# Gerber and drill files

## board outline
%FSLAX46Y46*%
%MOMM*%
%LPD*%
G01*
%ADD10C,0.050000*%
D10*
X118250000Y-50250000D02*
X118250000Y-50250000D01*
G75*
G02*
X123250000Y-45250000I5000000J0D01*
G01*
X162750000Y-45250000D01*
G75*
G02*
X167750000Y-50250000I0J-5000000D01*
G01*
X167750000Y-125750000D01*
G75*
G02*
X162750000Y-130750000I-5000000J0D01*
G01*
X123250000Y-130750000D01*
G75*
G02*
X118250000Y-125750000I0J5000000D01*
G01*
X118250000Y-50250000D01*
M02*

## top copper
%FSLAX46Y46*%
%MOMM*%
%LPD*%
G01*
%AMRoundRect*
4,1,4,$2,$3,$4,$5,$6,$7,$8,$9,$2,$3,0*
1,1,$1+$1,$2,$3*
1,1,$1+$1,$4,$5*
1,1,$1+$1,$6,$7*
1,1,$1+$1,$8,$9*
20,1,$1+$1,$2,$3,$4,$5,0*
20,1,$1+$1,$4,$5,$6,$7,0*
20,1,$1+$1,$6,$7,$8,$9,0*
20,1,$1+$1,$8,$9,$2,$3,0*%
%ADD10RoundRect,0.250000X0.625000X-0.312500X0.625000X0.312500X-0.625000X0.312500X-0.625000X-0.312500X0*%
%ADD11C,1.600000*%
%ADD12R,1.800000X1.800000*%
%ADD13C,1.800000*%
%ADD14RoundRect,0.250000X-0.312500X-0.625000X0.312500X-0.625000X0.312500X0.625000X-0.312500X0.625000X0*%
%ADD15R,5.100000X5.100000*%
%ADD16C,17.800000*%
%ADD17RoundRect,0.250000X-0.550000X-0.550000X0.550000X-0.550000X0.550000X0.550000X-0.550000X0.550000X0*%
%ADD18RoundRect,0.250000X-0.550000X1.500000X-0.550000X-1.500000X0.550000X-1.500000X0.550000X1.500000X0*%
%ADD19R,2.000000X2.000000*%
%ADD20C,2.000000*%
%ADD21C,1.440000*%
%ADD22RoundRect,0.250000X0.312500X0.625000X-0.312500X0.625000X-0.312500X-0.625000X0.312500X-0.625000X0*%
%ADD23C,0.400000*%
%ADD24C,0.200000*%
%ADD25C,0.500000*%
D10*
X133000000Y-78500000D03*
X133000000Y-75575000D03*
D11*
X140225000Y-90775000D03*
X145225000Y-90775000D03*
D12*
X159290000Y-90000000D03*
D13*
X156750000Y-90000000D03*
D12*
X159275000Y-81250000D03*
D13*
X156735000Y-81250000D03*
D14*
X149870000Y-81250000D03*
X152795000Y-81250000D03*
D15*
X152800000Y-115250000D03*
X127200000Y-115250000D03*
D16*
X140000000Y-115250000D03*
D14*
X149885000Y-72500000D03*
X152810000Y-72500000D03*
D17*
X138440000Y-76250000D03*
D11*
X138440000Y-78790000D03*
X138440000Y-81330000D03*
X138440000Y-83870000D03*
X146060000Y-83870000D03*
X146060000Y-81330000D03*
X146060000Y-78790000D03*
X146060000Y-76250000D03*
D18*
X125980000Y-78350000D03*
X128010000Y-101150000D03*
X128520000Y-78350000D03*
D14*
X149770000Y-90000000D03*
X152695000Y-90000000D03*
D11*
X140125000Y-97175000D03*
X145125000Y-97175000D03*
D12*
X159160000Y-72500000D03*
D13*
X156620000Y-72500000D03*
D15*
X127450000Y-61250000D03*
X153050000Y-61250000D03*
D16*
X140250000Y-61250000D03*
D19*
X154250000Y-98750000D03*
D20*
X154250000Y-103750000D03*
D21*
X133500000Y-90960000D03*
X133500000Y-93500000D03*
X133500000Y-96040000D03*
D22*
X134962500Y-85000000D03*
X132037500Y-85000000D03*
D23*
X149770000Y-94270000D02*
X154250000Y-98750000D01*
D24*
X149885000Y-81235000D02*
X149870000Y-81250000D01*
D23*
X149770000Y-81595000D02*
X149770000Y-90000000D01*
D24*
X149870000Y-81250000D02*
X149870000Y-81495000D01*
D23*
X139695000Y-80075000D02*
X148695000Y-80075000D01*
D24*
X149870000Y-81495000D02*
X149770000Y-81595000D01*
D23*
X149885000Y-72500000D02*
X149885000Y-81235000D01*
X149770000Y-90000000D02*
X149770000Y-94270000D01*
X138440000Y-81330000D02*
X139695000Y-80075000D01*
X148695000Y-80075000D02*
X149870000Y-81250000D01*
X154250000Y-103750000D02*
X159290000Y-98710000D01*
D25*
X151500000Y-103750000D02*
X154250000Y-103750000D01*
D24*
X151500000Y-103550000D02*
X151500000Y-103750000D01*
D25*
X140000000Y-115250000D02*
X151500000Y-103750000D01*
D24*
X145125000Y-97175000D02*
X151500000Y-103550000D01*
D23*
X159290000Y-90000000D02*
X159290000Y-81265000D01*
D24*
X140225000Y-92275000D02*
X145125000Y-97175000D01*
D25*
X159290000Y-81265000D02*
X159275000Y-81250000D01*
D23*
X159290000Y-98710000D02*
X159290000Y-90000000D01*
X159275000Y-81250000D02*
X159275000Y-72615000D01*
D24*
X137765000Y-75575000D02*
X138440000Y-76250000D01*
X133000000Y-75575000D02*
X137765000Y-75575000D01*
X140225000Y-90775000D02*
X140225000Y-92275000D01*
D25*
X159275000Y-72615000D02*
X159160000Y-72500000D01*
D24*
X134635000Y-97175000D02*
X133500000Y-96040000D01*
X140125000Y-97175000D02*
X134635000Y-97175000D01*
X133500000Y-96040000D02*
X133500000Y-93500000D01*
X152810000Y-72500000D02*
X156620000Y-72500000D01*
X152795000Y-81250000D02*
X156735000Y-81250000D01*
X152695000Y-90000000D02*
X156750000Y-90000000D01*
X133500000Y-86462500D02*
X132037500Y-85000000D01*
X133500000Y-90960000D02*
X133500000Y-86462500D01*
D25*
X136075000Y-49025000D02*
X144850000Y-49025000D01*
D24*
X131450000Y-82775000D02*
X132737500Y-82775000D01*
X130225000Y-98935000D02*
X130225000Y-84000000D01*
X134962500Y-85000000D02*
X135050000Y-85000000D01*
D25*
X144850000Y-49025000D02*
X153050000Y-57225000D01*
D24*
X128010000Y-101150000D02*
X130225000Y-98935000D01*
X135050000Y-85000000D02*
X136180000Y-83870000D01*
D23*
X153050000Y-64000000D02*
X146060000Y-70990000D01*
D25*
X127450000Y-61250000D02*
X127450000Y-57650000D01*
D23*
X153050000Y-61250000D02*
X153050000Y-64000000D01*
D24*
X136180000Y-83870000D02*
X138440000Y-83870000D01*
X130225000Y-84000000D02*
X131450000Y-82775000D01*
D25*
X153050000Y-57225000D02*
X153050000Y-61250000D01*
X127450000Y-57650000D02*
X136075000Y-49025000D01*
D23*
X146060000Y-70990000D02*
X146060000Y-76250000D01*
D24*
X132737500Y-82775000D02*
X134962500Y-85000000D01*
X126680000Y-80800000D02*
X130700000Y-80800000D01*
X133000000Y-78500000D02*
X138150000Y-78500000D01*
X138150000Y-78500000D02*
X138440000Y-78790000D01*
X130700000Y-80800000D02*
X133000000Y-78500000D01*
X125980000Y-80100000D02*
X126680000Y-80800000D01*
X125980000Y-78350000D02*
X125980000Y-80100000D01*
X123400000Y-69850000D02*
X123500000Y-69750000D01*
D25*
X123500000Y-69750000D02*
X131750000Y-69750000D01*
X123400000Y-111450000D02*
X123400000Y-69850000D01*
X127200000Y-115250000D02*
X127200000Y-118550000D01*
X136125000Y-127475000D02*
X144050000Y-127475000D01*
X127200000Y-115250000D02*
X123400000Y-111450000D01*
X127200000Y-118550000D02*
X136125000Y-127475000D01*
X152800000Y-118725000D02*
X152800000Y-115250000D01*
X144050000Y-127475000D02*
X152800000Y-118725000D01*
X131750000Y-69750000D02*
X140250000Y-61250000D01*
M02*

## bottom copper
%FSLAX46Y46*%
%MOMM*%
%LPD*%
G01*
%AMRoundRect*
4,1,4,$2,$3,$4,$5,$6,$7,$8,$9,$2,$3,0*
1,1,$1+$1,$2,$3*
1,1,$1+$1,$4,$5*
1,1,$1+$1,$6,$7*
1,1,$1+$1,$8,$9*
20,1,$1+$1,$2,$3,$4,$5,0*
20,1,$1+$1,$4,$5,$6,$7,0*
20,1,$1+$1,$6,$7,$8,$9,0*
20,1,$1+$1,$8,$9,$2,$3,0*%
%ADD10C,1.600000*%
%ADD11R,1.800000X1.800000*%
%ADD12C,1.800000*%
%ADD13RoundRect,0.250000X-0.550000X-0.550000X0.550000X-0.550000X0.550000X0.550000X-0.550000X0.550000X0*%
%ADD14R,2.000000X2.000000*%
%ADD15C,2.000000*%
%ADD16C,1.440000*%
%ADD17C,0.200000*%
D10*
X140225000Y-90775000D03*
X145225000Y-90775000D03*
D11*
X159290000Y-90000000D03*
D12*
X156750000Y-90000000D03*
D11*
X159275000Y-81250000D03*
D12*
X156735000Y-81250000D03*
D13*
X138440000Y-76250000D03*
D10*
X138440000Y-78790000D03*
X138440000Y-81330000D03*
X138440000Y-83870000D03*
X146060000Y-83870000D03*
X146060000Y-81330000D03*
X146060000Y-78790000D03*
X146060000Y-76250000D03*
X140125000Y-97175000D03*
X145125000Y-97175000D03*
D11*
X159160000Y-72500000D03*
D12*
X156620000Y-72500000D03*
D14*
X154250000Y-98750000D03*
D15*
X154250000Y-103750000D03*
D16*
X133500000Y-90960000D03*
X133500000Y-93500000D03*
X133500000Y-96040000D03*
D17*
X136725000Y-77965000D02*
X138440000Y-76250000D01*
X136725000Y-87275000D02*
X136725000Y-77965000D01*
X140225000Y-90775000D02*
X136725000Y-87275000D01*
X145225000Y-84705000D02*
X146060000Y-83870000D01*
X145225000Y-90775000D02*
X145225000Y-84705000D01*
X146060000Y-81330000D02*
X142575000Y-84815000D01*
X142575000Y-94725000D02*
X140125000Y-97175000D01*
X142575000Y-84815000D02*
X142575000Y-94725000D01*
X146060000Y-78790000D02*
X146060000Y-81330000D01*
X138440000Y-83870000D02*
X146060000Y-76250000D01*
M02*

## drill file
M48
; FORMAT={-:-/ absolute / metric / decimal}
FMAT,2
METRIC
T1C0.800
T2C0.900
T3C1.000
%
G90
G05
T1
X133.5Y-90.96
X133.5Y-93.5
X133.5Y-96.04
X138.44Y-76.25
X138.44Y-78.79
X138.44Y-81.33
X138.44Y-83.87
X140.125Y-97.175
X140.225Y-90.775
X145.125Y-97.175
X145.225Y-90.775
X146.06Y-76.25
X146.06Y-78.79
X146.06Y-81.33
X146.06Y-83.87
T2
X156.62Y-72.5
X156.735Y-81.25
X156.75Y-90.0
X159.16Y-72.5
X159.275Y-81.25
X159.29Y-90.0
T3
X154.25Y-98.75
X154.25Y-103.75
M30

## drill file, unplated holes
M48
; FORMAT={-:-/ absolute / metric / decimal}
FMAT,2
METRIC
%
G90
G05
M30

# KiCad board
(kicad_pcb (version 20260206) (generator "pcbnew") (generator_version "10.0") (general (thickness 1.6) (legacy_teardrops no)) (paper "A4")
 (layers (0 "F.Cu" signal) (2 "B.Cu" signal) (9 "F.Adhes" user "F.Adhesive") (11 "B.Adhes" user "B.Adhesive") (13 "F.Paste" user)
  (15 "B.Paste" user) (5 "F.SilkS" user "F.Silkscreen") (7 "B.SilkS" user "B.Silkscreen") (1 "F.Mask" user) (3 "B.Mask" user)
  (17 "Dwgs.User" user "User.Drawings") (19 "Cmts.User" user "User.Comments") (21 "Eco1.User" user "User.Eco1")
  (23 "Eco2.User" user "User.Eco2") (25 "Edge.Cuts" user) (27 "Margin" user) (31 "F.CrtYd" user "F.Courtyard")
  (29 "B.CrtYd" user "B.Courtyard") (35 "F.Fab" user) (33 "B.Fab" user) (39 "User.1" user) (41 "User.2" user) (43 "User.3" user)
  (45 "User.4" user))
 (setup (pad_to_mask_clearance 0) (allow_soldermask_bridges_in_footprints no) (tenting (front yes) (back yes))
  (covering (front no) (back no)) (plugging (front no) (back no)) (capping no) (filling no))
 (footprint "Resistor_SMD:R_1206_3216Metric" (layer "F.Cu") (at 133 77.0375 90)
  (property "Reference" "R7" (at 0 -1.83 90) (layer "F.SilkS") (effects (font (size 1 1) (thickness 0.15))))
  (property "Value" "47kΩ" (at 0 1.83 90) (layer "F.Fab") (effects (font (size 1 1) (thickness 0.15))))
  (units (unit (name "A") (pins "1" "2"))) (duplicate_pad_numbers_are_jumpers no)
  (pad "1" smd roundrect (at -1.4625 0 90) (size 1.125 1.75) (layers "F.Cu" "F.Mask" "F.Paste") (roundrect_rratio 0.222222)
   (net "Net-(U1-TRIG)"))
  (pad "2" smd roundrect (at 1.4625 0 90) (size 1.125 1.75) (layers "F.Cu" "F.Mask" "F.Paste") (roundrect_rratio 0.222222) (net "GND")))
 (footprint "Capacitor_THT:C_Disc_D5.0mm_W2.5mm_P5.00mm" (layer "F.Cu") (at 140.225 90.775)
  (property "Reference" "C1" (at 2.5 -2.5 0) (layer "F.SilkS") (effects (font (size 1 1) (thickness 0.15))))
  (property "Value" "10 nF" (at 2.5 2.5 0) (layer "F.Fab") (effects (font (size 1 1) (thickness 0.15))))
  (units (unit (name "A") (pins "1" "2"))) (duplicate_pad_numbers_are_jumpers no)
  (pad "1" thru_hole circle (at 0 0) (size 1.6 1.6) (drill 0.8) (layers "*.Cu" "*.Mask") (remove_unused_layers no) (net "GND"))
  (pad "2" thru_hole circle (at 5 0) (size 1.6 1.6) (drill 0.8) (layers "*.Cu" "*.Mask") (remove_unused_layers no) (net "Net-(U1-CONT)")))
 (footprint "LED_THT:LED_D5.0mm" (layer "F.Cu") (at 159.29 90 180)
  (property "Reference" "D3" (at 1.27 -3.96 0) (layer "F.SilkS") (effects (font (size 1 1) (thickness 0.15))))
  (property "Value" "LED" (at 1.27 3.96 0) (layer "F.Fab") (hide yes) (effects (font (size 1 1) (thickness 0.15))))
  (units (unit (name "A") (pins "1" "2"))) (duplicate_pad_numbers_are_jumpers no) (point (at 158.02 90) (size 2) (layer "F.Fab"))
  (pad "1" thru_hole rect (at 0 0 180) (size 1.8 1.8) (drill 0.9) (layers "*.Cu" "*.Mask") (remove_unused_layers no) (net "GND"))
  (pad "2" thru_hole circle (at 2.54 0 180) (size 1.8 1.8) (drill 0.9) (layers "*.Cu" "*.Mask") (remove_unused_layers no) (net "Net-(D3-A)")))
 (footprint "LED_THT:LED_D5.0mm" (layer "F.Cu") (at 159.275 81.25 180)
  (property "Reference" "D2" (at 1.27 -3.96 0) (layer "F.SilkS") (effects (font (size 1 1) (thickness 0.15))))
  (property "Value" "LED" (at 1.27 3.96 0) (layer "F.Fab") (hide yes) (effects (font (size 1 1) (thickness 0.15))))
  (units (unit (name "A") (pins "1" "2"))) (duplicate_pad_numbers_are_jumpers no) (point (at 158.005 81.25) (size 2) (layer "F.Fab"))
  (pad "1" thru_hole rect (at 0 0 180) (size 1.8 1.8) (drill 0.9) (layers "*.Cu" "*.Mask") (remove_unused_layers no) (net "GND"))
  (pad "2" thru_hole circle (at 2.54 0 180) (size 1.8 1.8) (drill 0.9) (layers "*.Cu" "*.Mask") (remove_unused_layers no) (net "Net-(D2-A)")))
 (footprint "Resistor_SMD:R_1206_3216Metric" (layer "F.Cu") (at 151.3325 81.25)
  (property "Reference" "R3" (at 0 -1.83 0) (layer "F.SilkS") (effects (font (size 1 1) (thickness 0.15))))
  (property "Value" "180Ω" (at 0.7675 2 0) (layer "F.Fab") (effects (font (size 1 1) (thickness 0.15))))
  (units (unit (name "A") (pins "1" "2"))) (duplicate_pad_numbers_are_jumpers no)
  (pad "1" smd roundrect (at -1.4625 0) (size 1.125 1.75) (layers "F.Cu" "F.Mask" "F.Paste") (roundrect_rratio 0.222222) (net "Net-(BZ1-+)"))
  (pad "2" smd roundrect (at 1.4625 0) (size 1.125 1.75) (layers "F.Cu" "F.Mask" "F.Paste") (roundrect_rratio 0.222222) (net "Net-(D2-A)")))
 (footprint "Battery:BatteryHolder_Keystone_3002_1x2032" (layer "F.Cu") (at 140 115.25 180)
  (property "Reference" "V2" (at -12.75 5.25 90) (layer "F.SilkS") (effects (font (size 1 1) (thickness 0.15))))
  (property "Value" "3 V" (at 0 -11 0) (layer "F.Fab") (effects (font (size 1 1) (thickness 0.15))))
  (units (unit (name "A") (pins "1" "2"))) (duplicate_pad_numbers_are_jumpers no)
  (pad "1" smd rect (at -12.8 0 180) (size 5.1 5.1) (layers "F.Cu" "F.Mask" "F.Paste") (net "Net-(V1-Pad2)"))
  (pad "1" smd rect (at 12.8 0 180) (size 5.1 5.1) (layers "F.Cu" "F.Mask" "F.Paste") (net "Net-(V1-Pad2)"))
  (pad "2" smd circle (at 0 0 180) (size 17.8 17.8) (layers "F.Cu" "F.Mask") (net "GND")))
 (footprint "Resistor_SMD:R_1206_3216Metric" (layer "F.Cu") (at 151.3475 72.5)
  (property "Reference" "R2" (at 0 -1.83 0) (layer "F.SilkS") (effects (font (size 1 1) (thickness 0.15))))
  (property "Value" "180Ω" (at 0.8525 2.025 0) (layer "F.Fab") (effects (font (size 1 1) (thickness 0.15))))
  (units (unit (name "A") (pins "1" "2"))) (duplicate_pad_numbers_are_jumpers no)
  (pad "1" smd roundrect (at -1.4625 0) (size 1.125 1.75) (layers "F.Cu" "F.Mask" "F.Paste") (roundrect_rratio 0.222222) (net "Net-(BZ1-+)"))
  (pad "2" smd roundrect (at 1.4625 0) (size 1.125 1.75) (layers "F.Cu" "F.Mask" "F.Paste") (roundrect_rratio 0.222222) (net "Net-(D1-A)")))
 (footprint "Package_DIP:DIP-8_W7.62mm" (layer "F.Cu") (at 138.44 76.25)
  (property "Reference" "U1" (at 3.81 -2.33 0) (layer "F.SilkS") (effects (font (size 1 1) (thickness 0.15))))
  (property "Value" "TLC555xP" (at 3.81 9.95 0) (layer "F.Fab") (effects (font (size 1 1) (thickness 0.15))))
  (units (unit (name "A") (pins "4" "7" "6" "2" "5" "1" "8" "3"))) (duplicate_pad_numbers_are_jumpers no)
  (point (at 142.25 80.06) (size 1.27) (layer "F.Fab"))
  (pad "1" thru_hole roundrect (at 0 0) (size 1.6 1.6) (drill 0.8) (layers "*.Cu" "*.Mask") (remove_unused_layers no)
   (roundrect_rratio 0.15625) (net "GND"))
  (pad "2" thru_hole circle (at 0 2.54) (size 1.6 1.6) (drill 0.8) (layers "*.Cu" "*.Mask") (remove_unused_layers no) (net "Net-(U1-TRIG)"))
  (pad "3" thru_hole circle (at 0 5.08) (size 1.6 1.6) (drill 0.8) (layers "*.Cu" "*.Mask") (remove_unused_layers no) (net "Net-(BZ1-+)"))
  (pad "4" thru_hole circle (at 0 7.62) (size 1.6 1.6) (drill 0.8) (layers "*.Cu" "*.Mask") (remove_unused_layers no) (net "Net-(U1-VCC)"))
  (pad "5" thru_hole circle (at 7.62 7.62) (size 1.6 1.6) (drill 0.8) (layers "*.Cu" "*.Mask") (remove_unused_layers no)
   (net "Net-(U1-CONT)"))
  (pad "6" thru_hole circle (at 7.62 5.08) (size 1.6 1.6) (drill 0.8) (layers "*.Cu" "*.Mask") (remove_unused_layers no)
   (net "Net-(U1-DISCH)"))
  (pad "7" thru_hole circle (at 7.62 2.54) (size 1.6 1.6) (drill 0.8) (layers "*.Cu" "*.Mask") (remove_unused_layers no)
   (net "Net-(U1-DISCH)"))
  (pad "8" thru_hole circle (at 7.62 0) (size 1.6 1.6) (drill 0.8) (layers "*.Cu" "*.Mask") (remove_unused_layers no) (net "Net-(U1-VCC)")))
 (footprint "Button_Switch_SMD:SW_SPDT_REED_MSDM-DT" (layer "F.Cu") (at 128.01 89.75)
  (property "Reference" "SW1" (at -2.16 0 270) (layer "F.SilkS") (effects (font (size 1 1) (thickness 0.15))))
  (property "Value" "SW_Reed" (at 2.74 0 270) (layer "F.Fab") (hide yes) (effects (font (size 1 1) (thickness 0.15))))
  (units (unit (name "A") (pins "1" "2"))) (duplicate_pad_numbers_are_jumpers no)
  (pad "1" smd roundrect (at -2.03 -11.4 270) (size 3.5 1.6) (layers "F.Cu" "F.Mask" "F.Paste") (roundrect_rratio 0.15625)
   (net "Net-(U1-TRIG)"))
  (pad "2" smd roundrect (at 0 11.4 270) (size 3.5 1.6) (layers "F.Cu" "F.Mask" "F.Paste") (roundrect_rratio 0.15625) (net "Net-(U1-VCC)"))
  (pad "3" smd roundrect (at 0.51 -11.4 270) (size 3.5 1.6) (layers "F.Cu" "F.Mask" "F.Paste") (roundrect_rratio 0.15625)))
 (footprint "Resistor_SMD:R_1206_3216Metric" (layer "F.Cu") (at 151.2325 90)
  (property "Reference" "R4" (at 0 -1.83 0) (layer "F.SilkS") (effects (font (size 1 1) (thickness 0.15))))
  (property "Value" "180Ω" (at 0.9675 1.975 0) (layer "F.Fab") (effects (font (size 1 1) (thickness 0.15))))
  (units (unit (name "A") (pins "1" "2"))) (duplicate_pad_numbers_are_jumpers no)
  (pad "1" smd roundrect (at -1.4625 0) (size 1.125 1.75) (layers "F.Cu" "F.Mask" "F.Paste") (roundrect_rratio 0.222222) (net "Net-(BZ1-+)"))
  (pad "2" smd roundrect (at 1.4625 0) (size 1.125 1.75) (layers "F.Cu" "F.Mask" "F.Paste") (roundrect_rratio 0.222222) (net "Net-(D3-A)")))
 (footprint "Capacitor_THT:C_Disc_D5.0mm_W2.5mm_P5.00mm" (layer "F.Cu") (at 140.125 97.175)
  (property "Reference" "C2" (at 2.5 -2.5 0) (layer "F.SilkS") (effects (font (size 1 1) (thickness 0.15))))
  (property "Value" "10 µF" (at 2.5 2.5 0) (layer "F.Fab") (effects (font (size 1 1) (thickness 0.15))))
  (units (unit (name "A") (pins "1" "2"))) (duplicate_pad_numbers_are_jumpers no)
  (pad "1" thru_hole circle (at 0 0) (size 1.6 1.6) (drill 0.8) (layers "*.Cu" "*.Mask") (remove_unused_layers no) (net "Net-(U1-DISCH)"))
  (pad "2" thru_hole circle (at 5 0) (size 1.6 1.6) (drill 0.8) (layers "*.Cu" "*.Mask") (remove_unused_layers no) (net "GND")))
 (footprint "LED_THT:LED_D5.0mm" (layer "F.Cu") (at 159.16 72.5 180)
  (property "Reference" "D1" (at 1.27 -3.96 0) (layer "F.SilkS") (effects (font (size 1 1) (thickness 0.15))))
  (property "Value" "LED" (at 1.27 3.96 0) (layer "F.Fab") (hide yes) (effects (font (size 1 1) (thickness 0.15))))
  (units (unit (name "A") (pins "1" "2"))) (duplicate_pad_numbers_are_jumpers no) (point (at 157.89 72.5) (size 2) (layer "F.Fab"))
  (pad "1" thru_hole rect (at 0 0 180) (size 1.8 1.8) (drill 0.9) (layers "*.Cu" "*.Mask") (remove_unused_layers no) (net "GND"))
  (pad "2" thru_hole circle (at 2.54 0 180) (size 1.8 1.8) (drill 0.9) (layers "*.Cu" "*.Mask") (remove_unused_layers no) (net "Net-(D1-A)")))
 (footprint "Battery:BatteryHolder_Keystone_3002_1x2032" (layer "F.Cu") (at 140.25 61.25)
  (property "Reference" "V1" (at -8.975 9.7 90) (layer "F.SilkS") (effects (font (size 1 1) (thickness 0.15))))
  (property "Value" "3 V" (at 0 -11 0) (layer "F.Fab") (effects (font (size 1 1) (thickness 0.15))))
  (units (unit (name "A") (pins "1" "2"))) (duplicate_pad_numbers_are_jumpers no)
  (pad "1" smd rect (at -12.8 0) (size 5.1 5.1) (layers "F.Cu" "F.Mask" "F.Paste") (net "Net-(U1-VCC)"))
  (pad "1" smd rect (at 12.8 0) (size 5.1 5.1) (layers "F.Cu" "F.Mask" "F.Paste") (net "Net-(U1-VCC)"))
  (pad "2" smd circle (at 0 0) (size 17.8 17.8) (layers "F.Cu" "F.Mask") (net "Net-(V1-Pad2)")))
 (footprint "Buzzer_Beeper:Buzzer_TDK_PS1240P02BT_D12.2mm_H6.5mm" (layer "F.Cu") (at 154.25 98.75 -90)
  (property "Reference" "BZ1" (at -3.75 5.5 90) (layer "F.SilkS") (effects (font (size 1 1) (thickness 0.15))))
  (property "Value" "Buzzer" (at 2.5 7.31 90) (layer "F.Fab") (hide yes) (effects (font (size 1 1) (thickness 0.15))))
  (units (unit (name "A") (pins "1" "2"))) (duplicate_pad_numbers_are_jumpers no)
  (pad "1" thru_hole rect (at 0 0 270) (size 2 2) (drill 1) (layers "*.Cu" "*.Mask") (remove_unused_layers no) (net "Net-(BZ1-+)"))
  (pad "2" thru_hole circle (at 5 0 270) (size 2 2) (drill 1) (layers "*.Cu" "*.Mask") (remove_unused_layers no) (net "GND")))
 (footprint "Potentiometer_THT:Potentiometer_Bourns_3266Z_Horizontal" (layer "F.Cu") (at 133.5 90.96 90)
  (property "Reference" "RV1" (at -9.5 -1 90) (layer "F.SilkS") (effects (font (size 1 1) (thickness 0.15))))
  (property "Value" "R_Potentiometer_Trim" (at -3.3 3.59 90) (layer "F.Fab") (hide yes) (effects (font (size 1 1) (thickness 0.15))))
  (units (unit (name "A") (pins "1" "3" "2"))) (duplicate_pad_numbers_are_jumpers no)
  (pad "1" thru_hole circle (at 0 0 90) (size 1.44 1.44) (drill 0.8) (layers "*.Cu" "*.Mask") (remove_unused_layers no)
   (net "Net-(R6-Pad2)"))
  (pad "2" thru_hole circle (at -2.54 0 90) (size 1.44 1.44) (drill 0.8) (layers "*.Cu" "*.Mask") (remove_unused_layers no)
   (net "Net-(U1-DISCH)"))
  (pad "3" thru_hole circle (at -5.08 0 90) (size 1.44 1.44) (drill 0.8) (layers "*.Cu" "*.Mask") (remove_unused_layers no)
   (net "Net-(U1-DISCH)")))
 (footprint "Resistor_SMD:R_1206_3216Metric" (layer "F.Cu") (at 133.5 85 180)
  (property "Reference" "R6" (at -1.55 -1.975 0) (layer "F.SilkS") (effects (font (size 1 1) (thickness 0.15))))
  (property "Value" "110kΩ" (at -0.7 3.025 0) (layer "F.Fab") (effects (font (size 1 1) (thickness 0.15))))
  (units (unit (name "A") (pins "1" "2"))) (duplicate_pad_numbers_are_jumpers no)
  (pad "1" smd roundrect (at -1.4625 0 180) (size 1.125 1.75) (layers "F.Cu" "F.Mask" "F.Paste") (roundrect_rratio 0.222222)
   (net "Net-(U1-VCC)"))
  (pad "2" smd roundrect (at 1.4625 0 180) (size 1.125 1.75) (layers "F.Cu" "F.Mask" "F.Paste") (roundrect_rratio 0.222222)
   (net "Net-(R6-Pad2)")))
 (gr_rect (start 118.25 45.25) (end 167.75 130.75) (radius 5) (stroke (width 0.05) (type solid)) (fill no) (layer "Edge.Cuts"))
 (segment (start 126.68 80.8) (end 130.7 80.8) (width 0.2) (layer "F.Cu") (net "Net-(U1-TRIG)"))
 (segment (start 133 78.5) (end 138.15 78.5) (width 0.2) (layer "F.Cu") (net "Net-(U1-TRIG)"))
 (segment (start 138.15 78.5) (end 138.44 78.79) (width 0.2) (layer "F.Cu") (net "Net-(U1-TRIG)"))
 (segment (start 130.7 80.8) (end 133 78.5) (width 0.2) (layer "F.Cu") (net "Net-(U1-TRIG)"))
 (segment (start 125.98 80.1) (end 126.68 80.8) (width 0.2) (layer "F.Cu") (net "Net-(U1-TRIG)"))
 (segment (start 125.98 78.35) (end 125.98 80.1) (width 0.2) (layer "F.Cu") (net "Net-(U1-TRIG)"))
 (segment (start 154.25 103.75) (end 159.29 98.71) (width 0.4) (layer "F.Cu") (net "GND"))
 (segment (start 151.5 103.75) (end 154.25 103.75) (width 0.5) (layer "F.Cu") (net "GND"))
 (segment (start 151.5 103.55) (end 151.5 103.75) (width 0.2) (layer "F.Cu") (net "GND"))
 (segment (start 140 115.25) (end 151.5 103.75) (width 0.5) (layer "F.Cu") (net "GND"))
 (segment (start 145.125 97.175) (end 151.5 103.55) (width 0.2) (layer "F.Cu") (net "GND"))
 (segment (start 159.29 90) (end 159.29 81.265) (width 0.4) (layer "F.Cu") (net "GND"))
 (segment (start 140.225 92.275) (end 145.125 97.175) (width 0.2) (layer "F.Cu") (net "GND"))
 (segment (start 159.29 81.265) (end 159.275 81.25) (width 0.5) (layer "F.Cu") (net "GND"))
 (segment (start 159.29 98.71) (end 159.29 90) (width 0.4) (layer "F.Cu") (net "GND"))
 (segment (start 159.275 81.25) (end 159.275 72.615) (width 0.4) (layer "F.Cu") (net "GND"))
 (segment (start 137.765 75.575) (end 138.44 76.25) (width 0.2) (layer "F.Cu") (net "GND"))
 (segment (start 133 75.575) (end 137.765 75.575) (width 0.2) (layer "F.Cu") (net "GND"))
 (segment (start 140.225 90.775) (end 140.225 92.275) (width 0.2) (layer "F.Cu") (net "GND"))
 (segment (start 159.275 72.615) (end 159.16 72.5) (width 0.5) (layer "F.Cu") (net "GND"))
 (segment (start 136.725 77.965) (end 138.44 76.25) (width 0.2) (layer "B.Cu") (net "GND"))
 (segment (start 136.725 87.275) (end 136.725 77.965) (width 0.2) (layer "B.Cu") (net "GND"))
 (segment (start 140.225 90.775) (end 136.725 87.275) (width 0.2) (layer "B.Cu") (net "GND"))
 (segment (start 145.225 84.705) (end 146.06 83.87) (width 0.2) (layer "B.Cu") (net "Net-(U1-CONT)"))
 (segment (start 145.225 90.775) (end 145.225 84.705) (width 0.2) (layer "B.Cu") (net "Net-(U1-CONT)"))
 (segment (start 152.695 90) (end 156.75 90) (width 0.2) (layer "F.Cu") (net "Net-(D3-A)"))
 (segment (start 152.795 81.25) (end 156.735 81.25) (width 0.2) (layer "F.Cu") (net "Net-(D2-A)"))
 (segment (start 149.77 94.27) (end 154.25 98.75) (width 0.4) (layer "F.Cu") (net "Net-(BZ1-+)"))
 (segment (start 149.885 81.235) (end 149.87 81.25) (width 0.2) (layer "F.Cu") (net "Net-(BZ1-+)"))
 (segment (start 149.77 81.595) (end 149.77 90) (width 0.4) (layer "F.Cu") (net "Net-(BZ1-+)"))
 (segment (start 149.87 81.25) (end 149.87 81.495) (width 0.2) (layer "F.Cu") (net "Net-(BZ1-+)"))
 (segment (start 139.695 80.075) (end 148.695 80.075) (width 0.4) (layer "F.Cu") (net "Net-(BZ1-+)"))
 (segment (start 149.87 81.495) (end 149.77 81.595) (width 0.2) (layer "F.Cu") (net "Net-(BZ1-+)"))
 (segment (start 149.885 72.5) (end 149.885 81.235) (width 0.4) (layer "F.Cu") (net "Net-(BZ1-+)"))
 (segment (start 149.77 90) (end 149.77 94.27) (width 0.4) (layer "F.Cu") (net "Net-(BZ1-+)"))
 (segment (start 138.44 81.33) (end 139.695 80.075) (width 0.4) (layer "F.Cu") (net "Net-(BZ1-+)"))
 (segment (start 148.695 80.075) (end 149.87 81.25) (width 0.4) (layer "F.Cu") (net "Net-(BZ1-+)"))
 (segment (start 123.4 69.85) (end 123.5 69.75) (width 0.2) (layer "F.Cu") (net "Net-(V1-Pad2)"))
 (segment (start 123.5 69.75) (end 131.75 69.75) (width 0.5) (layer "F.Cu") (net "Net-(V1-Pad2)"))
 (segment (start 123.4 111.45) (end 123.4 69.85) (width 0.5) (layer "F.Cu") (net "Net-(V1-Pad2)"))
 (segment (start 127.2 115.25) (end 127.2 118.55) (width 0.5) (layer "F.Cu") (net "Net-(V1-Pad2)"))
 (segment (start 136.125 127.475) (end 144.05 127.475) (width 0.5) (layer "F.Cu") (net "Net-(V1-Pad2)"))
 (segment (start 127.2 115.25) (end 123.4 111.45) (width 0.5) (layer "F.Cu") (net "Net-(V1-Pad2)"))
 (segment (start 127.2 118.55) (end 136.125 127.475) (width 0.5) (layer "F.Cu") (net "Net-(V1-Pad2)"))
 (segment (start 152.8 118.725) (end 152.8 115.25) (width 0.5) (layer "F.Cu") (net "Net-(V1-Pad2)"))
 (segment (start 144.05 127.475) (end 152.8 118.725) (width 0.5) (layer "F.Cu") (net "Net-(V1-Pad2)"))
 (segment (start 131.75 69.75) (end 140.25 61.25) (width 0.5) (layer "F.Cu") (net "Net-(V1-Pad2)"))
 (segment (start 152.81 72.5) (end 156.62 72.5) (width 0.2) (layer "F.Cu") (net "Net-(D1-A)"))
 (segment (start 136.075 49.025) (end 144.85 49.025) (width 0.5) (layer "F.Cu") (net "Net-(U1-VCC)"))
 (segment (start 131.45 82.775) (end 132.7375 82.775) (width 0.2) (layer "F.Cu") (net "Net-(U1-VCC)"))
 (segment (start 130.225 98.935) (end 130.225 84) (width 0.2) (layer "F.Cu") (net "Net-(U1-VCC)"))
 (segment (start 134.9625 85) (end 135.05 85) (width 0.2) (layer "F.Cu") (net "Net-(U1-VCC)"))
 (segment (start 144.85 49.025) (end 153.05 57.225) (width 0.5) (layer "F.Cu") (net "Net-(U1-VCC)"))
 (segment (start 128.01 101.15) (end 130.225 98.935) (width 0.2) (layer "F.Cu") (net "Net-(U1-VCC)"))
 (segment (start 135.05 85) (end 136.18 83.87) (width 0.2) (layer "F.Cu") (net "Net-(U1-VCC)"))
 (segment (start 153.05 64) (end 146.06 70.99) (width 0.4) (layer "F.Cu") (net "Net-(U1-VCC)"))
 (segment (start 127.45 61.25) (end 127.45 57.65) (width 0.5) (layer "F.Cu") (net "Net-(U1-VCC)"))
 (segment (start 153.05 61.25) (end 153.05 64) (width 0.4) (layer "F.Cu") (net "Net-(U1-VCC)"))
 (segment (start 136.18 83.87) (end 138.44 83.87) (width 0.2) (layer "F.Cu") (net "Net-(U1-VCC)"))
 (segment (start 130.225 84) (end 131.45 82.775) (width 0.2) (layer "F.Cu") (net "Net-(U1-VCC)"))
 (segment (start 153.05 57.225) (end 153.05 61.25) (width 0.5) (layer "F.Cu") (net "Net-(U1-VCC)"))
 (segment (start 127.45 57.65) (end 136.075 49.025) (width 0.5) (layer "F.Cu") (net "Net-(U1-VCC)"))
 (segment (start 146.06 70.99) (end 146.06 76.25) (width 0.4) (layer "F.Cu") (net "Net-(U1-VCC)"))
 (segment (start 132.7375 82.775) (end 134.9625 85) (width 0.2) (layer "F.Cu") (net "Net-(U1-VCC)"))
 (segment (start 138.44 83.87) (end 146.06 76.25) (width 0.2) (layer "B.Cu") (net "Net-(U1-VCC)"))
 (segment (start 134.635 97.175) (end 133.5 96.04) (width 0.2) (layer "F.Cu") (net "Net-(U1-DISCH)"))
 (segment (start 140.125 97.175) (end 134.635 97.175) (width 0.2) (layer "F.Cu") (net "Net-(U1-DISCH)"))
 (segment (start 133.5 96.04) (end 133.5 93.5) (width 0.2) (layer "F.Cu") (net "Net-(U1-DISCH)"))
 (segment (start 146.06 81.33) (end 142.575 84.815) (width 0.2) (layer "B.Cu") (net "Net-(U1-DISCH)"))
 (segment (start 142.575 94.725) (end 140.125 97.175) (width 0.2) (layer "B.Cu") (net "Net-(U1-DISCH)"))
 (segment (start 142.575 84.815) (end 142.575 94.725) (width 0.2) (layer "B.Cu") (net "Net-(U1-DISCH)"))
 (segment (start 146.06 78.79) (end 146.06 81.33) (width 0.2) (layer "B.Cu") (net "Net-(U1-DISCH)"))
 (segment (start 133.5 86.4625) (end 132.0375 85) (width 0.2) (layer "F.Cu") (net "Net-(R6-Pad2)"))
 (segment (start 133.5 90.96) (end 133.5 86.4625) (width 0.2) (layer "F.Cu") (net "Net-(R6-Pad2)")))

